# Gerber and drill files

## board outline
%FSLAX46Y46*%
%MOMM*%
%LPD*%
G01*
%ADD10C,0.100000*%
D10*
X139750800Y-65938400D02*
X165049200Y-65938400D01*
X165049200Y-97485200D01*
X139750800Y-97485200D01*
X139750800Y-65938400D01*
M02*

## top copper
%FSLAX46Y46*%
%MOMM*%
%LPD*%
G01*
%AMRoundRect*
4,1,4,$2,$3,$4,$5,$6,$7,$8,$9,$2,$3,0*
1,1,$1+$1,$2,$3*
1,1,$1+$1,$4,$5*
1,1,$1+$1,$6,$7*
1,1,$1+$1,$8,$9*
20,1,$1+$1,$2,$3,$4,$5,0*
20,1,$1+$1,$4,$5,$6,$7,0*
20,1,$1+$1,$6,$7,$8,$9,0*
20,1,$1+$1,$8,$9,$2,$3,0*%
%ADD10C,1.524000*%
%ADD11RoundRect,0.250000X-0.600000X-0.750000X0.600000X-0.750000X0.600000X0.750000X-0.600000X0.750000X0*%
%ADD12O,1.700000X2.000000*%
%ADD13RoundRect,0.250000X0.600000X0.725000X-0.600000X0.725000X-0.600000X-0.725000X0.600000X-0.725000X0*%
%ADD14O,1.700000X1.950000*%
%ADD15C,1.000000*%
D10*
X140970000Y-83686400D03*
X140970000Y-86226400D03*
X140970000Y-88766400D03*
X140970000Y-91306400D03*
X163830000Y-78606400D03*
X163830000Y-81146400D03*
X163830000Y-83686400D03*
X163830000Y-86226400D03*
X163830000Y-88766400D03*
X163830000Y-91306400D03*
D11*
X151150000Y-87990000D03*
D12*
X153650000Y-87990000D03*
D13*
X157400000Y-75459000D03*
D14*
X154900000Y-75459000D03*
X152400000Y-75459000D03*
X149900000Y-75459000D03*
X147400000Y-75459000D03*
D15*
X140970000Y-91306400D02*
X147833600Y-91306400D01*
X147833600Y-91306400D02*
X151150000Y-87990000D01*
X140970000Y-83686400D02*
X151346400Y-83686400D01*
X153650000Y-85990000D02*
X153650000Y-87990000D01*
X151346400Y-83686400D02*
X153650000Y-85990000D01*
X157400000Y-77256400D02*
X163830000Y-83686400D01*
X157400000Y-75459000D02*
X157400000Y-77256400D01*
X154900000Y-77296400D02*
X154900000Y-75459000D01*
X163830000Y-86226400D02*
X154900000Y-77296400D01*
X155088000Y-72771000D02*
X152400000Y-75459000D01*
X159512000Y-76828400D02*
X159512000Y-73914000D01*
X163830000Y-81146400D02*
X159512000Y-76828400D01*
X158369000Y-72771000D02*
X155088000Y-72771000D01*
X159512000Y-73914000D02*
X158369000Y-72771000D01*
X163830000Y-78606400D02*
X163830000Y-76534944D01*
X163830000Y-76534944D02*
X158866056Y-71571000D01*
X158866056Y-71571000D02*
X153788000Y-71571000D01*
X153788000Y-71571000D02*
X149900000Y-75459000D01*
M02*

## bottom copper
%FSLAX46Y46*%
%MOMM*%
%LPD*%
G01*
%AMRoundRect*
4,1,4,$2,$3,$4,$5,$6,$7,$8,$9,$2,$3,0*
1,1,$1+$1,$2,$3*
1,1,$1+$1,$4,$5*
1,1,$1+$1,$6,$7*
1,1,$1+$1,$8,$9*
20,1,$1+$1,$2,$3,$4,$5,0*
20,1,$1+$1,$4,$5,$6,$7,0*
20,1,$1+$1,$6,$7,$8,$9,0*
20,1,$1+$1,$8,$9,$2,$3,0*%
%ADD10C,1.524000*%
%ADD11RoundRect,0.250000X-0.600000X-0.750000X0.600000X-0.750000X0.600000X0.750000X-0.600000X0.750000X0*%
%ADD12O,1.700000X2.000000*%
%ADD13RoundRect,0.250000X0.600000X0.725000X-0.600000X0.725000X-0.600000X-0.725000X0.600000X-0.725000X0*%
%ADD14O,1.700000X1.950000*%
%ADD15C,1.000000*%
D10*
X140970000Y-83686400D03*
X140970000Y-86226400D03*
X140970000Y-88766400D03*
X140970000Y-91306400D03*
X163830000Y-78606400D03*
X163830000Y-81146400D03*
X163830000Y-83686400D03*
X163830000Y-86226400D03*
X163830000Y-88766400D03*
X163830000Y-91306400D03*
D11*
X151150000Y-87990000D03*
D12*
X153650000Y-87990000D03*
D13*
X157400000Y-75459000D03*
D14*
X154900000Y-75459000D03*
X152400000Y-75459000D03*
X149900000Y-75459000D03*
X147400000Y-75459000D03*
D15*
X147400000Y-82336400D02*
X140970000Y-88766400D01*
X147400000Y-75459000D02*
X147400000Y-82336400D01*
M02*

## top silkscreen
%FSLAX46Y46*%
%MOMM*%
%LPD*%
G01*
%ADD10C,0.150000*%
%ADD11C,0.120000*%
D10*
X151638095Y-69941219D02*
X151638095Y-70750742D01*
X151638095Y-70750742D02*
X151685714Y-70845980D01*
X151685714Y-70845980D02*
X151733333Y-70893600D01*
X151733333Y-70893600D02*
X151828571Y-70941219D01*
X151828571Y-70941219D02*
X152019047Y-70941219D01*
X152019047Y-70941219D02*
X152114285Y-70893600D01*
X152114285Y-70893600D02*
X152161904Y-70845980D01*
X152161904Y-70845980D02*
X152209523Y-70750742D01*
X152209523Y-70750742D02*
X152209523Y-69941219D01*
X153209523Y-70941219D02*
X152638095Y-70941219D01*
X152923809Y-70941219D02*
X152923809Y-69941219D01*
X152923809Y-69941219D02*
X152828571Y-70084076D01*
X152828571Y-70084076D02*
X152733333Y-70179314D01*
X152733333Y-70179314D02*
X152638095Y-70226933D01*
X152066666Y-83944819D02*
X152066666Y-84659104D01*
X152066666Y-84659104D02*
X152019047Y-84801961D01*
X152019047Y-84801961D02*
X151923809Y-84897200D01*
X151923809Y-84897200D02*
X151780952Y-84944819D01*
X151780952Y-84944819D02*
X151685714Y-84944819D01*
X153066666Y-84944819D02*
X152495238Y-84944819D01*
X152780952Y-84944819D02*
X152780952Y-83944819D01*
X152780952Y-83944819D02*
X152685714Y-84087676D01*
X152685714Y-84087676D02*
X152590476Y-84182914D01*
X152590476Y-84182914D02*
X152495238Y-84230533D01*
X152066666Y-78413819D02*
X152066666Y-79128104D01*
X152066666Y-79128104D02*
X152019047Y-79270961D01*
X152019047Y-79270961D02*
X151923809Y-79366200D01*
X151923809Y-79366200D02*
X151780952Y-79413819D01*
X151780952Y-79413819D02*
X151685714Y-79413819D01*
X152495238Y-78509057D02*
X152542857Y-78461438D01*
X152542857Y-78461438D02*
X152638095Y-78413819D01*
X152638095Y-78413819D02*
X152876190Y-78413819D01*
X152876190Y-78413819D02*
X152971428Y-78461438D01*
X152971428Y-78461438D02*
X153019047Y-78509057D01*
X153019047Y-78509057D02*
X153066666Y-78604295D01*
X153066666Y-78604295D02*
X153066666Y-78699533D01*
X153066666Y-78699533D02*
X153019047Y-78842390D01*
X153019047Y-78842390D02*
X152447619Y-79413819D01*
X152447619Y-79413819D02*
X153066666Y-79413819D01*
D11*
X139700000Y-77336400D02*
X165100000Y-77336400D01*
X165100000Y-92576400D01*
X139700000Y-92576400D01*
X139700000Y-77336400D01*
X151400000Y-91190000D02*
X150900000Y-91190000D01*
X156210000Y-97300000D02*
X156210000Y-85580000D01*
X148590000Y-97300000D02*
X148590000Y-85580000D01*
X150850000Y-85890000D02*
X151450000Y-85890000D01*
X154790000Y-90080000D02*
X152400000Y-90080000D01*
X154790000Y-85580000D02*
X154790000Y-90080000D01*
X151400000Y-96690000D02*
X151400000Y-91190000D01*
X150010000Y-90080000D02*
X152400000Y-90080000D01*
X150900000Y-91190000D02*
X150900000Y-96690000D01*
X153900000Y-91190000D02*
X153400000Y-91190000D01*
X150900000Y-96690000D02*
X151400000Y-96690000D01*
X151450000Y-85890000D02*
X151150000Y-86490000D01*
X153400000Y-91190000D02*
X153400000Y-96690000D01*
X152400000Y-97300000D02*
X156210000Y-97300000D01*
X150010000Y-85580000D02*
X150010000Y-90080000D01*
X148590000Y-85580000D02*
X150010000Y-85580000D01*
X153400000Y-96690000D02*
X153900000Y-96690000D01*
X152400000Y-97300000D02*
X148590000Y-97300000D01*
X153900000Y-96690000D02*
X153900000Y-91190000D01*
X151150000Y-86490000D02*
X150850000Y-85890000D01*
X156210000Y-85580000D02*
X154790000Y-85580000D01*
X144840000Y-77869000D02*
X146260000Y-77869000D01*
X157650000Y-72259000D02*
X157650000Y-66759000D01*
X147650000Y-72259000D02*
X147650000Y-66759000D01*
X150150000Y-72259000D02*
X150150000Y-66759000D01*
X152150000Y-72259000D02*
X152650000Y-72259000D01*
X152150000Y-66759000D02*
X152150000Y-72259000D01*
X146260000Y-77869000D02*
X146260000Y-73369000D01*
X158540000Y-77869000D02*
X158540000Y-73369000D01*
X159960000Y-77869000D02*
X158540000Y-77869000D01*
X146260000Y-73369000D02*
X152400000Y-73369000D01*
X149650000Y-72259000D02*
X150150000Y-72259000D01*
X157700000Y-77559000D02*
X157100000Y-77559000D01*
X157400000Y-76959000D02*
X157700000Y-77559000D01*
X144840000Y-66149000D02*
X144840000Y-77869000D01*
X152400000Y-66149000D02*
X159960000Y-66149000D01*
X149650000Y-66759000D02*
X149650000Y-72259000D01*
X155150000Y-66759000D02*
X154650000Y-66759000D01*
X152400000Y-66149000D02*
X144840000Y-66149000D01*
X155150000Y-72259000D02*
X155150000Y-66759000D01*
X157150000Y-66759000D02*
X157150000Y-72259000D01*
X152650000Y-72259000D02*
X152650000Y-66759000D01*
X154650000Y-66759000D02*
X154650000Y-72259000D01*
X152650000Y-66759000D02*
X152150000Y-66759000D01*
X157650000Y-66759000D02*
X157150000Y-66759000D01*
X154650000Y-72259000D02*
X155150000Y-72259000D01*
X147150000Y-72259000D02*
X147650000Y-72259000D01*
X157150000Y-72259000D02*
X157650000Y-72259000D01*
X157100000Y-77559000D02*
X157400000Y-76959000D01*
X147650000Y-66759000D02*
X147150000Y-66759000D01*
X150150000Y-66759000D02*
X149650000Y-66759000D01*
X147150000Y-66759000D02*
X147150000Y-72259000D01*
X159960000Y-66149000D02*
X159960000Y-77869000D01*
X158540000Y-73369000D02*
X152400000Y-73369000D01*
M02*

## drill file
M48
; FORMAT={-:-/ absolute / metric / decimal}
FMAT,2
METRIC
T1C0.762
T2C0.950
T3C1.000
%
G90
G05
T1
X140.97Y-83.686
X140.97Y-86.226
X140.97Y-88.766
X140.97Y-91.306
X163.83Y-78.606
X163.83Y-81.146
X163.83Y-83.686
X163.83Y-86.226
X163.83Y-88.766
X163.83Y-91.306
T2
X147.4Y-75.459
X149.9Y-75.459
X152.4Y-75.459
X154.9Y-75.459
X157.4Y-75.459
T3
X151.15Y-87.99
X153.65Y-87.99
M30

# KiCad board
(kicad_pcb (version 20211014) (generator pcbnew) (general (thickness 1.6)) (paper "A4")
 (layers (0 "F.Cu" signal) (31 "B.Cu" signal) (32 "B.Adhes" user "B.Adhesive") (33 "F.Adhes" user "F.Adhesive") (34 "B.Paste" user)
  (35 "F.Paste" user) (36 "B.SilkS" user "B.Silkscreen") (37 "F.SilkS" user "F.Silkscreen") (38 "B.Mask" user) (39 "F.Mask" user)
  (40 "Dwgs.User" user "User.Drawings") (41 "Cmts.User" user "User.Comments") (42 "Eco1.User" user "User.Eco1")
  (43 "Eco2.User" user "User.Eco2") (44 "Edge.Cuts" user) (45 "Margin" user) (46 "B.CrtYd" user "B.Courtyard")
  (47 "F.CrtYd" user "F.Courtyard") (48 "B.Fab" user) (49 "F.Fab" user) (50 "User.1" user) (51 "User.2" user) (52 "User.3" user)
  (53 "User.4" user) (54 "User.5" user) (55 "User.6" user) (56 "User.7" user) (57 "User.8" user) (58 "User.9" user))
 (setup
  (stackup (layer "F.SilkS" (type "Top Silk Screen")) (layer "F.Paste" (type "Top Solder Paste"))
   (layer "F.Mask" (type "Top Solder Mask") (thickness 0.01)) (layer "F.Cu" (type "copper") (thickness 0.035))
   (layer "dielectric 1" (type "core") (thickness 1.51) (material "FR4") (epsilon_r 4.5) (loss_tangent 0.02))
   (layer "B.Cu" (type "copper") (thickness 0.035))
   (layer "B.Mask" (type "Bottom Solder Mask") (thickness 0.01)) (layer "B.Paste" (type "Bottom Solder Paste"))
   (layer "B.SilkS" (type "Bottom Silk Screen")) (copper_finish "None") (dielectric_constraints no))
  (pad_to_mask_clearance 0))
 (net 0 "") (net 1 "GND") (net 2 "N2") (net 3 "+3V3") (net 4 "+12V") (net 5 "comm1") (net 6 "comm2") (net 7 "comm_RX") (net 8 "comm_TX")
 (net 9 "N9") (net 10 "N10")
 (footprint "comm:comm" (layer "F.Cu") (at 152.4 70.9864)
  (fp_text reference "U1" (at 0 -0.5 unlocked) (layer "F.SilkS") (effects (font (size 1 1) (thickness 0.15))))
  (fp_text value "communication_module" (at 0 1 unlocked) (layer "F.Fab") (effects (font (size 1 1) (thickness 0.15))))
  (fp_rect (start -12.7 21.59) (end 12.7 6.35) (layer "F.SilkS") (width 0.12) (fill none))
  (pad "1" thru_hole circle (at -11.43 12.7) (size 1.524 1.524) (drill 0.762) (layers *.Cu *.Mask) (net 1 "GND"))
  (pad "2" thru_hole circle (at -11.43 15.24) (size 1.524 1.524) (drill 0.762) (layers *.Cu *.Mask) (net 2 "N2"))
  (pad "3" thru_hole circle (at -11.43 17.78) (size 1.524 1.524) (drill 0.762) (layers *.Cu *.Mask) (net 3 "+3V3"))
  (pad "4" thru_hole circle (at -11.43 20.32) (size 1.524 1.524) (drill 0.762) (layers *.Cu *.Mask) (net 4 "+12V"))
  (pad "5" thru_hole circle (at 11.43 7.62) (size 1.524 1.524) (drill 0.762) (layers *.Cu *.Mask) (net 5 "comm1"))
  (pad "6" thru_hole circle (at 11.43 10.16) (size 1.524 1.524) (drill 0.762) (layers *.Cu *.Mask) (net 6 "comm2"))
  (pad "7" thru_hole circle (at 11.43 12.7) (size 1.524 1.524) (drill 0.762) (layers *.Cu *.Mask) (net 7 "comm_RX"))
  (pad "8" thru_hole circle (at 11.43 15.24) (size 1.524 1.524) (drill 0.762) (layers *.Cu *.Mask) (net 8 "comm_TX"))
  (pad "9" thru_hole circle (at 11.43 17.78) (size 1.524 1.524) (drill 0.762) (layers *.Cu *.Mask) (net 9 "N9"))
  (pad "10" thru_hole circle (at 11.43 20.32) (size 1.524 1.524) (drill 0.762) (layers *.Cu *.Mask) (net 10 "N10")))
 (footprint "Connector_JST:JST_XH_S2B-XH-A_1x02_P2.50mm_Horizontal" (layer "F.Cu") (at 151.15 87.99)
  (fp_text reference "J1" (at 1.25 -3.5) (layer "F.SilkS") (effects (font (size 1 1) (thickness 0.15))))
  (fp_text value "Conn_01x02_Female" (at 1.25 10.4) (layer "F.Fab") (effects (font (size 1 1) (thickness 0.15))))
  (fp_line (start 0.25 3.2) (end -0.25 3.2) (layer "F.SilkS") (width 0.12))
  (fp_line (start 5.06 9.31) (end 5.06 -2.41) (layer "F.SilkS") (width 0.12))
  (fp_line (start -2.56 9.31) (end -2.56 -2.41) (layer "F.SilkS") (width 0.12))
  (fp_line (start -0.3 -2.1) (end 0.3 -2.1) (layer "F.SilkS") (width 0.12))
  (fp_line (start 3.64 2.09) (end 1.25 2.09) (layer "F.SilkS") (width 0.12))
  (fp_line (start 3.64 -2.41) (end 3.64 2.09) (layer "F.SilkS") (width 0.12))
  (fp_line (start 0.25 8.7) (end 0.25 3.2) (layer "F.SilkS") (width 0.12))
  (fp_line (start -1.14 2.09) (end 1.25 2.09) (layer "F.SilkS") (width 0.12))
  (fp_line (start -0.25 3.2) (end -0.25 8.7) (layer "F.SilkS") (width 0.12))
  (fp_line (start 2.75 3.2) (end 2.25 3.2) (layer "F.SilkS") (width 0.12))
  (fp_line (start -0.25 8.7) (end 0.25 8.7) (layer "F.SilkS") (width 0.12))
  (fp_line (start 0.3 -2.1) (end 0 -1.5) (layer "F.SilkS") (width 0.12))
  (fp_line (start 2.25 3.2) (end 2.25 8.7) (layer "F.SilkS") (width 0.12))
  (fp_line (start 1.25 9.31) (end 5.06 9.31) (layer "F.SilkS") (width 0.12))
  (fp_line (start -1.14 -2.41) (end -1.14 2.09) (layer "F.SilkS") (width 0.12))
  (fp_line (start -2.56 -2.41) (end -1.14 -2.41) (layer "F.SilkS") (width 0.12))
  (fp_line (start 2.25 8.7) (end 2.75 8.7) (layer "F.SilkS") (width 0.12))
  (fp_line (start 1.25 9.31) (end -2.56 9.31) (layer "F.SilkS") (width 0.12))
  (fp_line (start 2.75 8.7) (end 2.75 3.2) (layer "F.SilkS") (width 0.12))
  (fp_line (start 0 -1.5) (end -0.3 -2.1) (layer "F.SilkS") (width 0.12))
  (fp_line (start 5.06 -2.41) (end 3.64 -2.41) (layer "F.SilkS") (width 0.12))
  (pad "1" thru_hole roundrect (at 0 0) (size 1.7 2) (drill 1) (layers *.Cu *.Mask) (roundrect_rratio 0.147059) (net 4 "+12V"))
  (pad "2" thru_hole oval (at 2.5 0) (size 1.7 2) (drill 1) (layers *.Cu *.Mask) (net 1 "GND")))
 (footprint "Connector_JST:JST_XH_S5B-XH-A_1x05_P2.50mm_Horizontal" (layer "F.Cu") (at 157.4 75.459 180)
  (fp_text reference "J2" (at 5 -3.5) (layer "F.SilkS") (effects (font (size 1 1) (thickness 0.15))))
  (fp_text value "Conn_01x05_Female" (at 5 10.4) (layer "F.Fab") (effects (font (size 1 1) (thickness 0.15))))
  (fp_line (start 12.56 -2.41) (end 11.14 -2.41) (layer "F.SilkS") (width 0.12))
  (fp_line (start -0.25 3.2) (end -0.25 8.7) (layer "F.SilkS") (width 0.12))
  (fp_line (start 9.75 3.2) (end 9.75 8.7) (layer "F.SilkS") (width 0.12))
  (fp_line (start 7.25 3.2) (end 7.25 8.7) (layer "F.SilkS") (width 0.12))
  (fp_line (start 5.25 3.2) (end 4.75 3.2) (layer "F.SilkS") (width 0.12))
  (fp_line (start 5.25 8.7) (end 5.25 3.2) (layer "F.SilkS") (width 0.12))
  (fp_line (start 11.14 -2.41) (end 11.14 2.09) (layer "F.SilkS") (width 0.12))
  (fp_line (start -1.14 -2.41) (end -1.14 2.09) (layer "F.SilkS") (width 0.12))
  (fp_line (start -2.56 -2.41) (end -1.14 -2.41) (layer "F.SilkS") (width 0.12))
  (fp_line (start 11.14 2.09) (end 5 2.09) (layer "F.SilkS") (width 0.12))
  (fp_line (start 7.75 3.2) (end 7.25 3.2) (layer "F.SilkS") (width 0.12))
  (fp_line (start -0.3 -2.1) (end 0.3 -2.1) (layer "F.SilkS") (width 0.12))
  (fp_line (start 0 -1.5) (end -0.3 -2.1) (layer "F.SilkS") (width 0.12))
  (fp_line (start 12.56 9.31) (end 12.56 -2.41) (layer "F.SilkS") (width 0.12))
  (fp_line (start 5 9.31) (end -2.56 9.31) (layer "F.SilkS") (width 0.12))
  (fp_line (start 7.75 8.7) (end 7.75 3.2) (layer "F.SilkS") (width 0.12))
  (fp_line (start 2.25 8.7) (end 2.75 8.7) (layer "F.SilkS") (width 0.12))
  (fp_line (start 5 9.31) (end 12.56 9.31) (layer "F.SilkS") (width 0.12))
  (fp_line (start 2.25 3.2) (end 2.25 8.7) (layer "F.SilkS") (width 0.12))
  (fp_line (start 0.25 8.7) (end 0.25 3.2) (layer "F.SilkS") (width 0.12))
  (fp_line (start 4.75 3.2) (end 4.75 8.7) (layer "F.SilkS") (width 0.12))
  (fp_line (start 2.75 8.7) (end 2.75 3.2) (layer "F.SilkS") (width 0.12))
  (fp_line (start 4.75 8.7) (end 5.25 8.7) (layer "F.SilkS") (width 0.12))
  (fp_line (start -0.25 8.7) (end 0.25 8.7) (layer "F.SilkS") (width 0.12))
  (fp_line (start 2.75 3.2) (end 2.25 3.2) (layer "F.SilkS") (width 0.12))
  (fp_line (start 10.25 3.2) (end 9.75 3.2) (layer "F.SilkS") (width 0.12))
  (fp_line (start 0.25 3.2) (end -0.25 3.2) (layer "F.SilkS") (width 0.12))
  (fp_line (start 0.3 -2.1) (end 0 -1.5) (layer "F.SilkS") (width 0.12))
  (fp_line (start 9.75 8.7) (end 10.25 8.7) (layer "F.SilkS") (width 0.12))
  (fp_line (start 7.25 8.7) (end 7.75 8.7) (layer "F.SilkS") (width 0.12))
  (fp_line (start 10.25 8.7) (end 10.25 3.2) (layer "F.SilkS") (width 0.12))
  (fp_line (start -2.56 9.31) (end -2.56 -2.41) (layer "F.SilkS") (width 0.12))
  (fp_line (start -1.14 2.09) (end 5 2.09) (layer "F.SilkS") (width 0.12))
  (pad "1" thru_hole roundrect (at 0 0 180) (size 1.7 1.95) (drill 0.95) (layers *.Cu *.Mask) (roundrect_rratio 0.147059) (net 7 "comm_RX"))
  (pad "2" thru_hole oval (at 2.5 0 180) (size 1.7 1.95) (drill 0.95) (layers *.Cu *.Mask) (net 8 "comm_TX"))
  (pad "3" thru_hole oval (at 5 0 180) (size 1.7 1.95) (drill 0.95) (layers *.Cu *.Mask) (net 6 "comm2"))
  (pad "4" thru_hole oval (at 7.5 0 180) (size 1.7 1.95) (drill 0.95) (layers *.Cu *.Mask) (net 5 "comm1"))
  (pad "5" thru_hole oval (at 10 0 180) (size 1.7 1.95) (drill 0.95) (layers *.Cu *.Mask) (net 3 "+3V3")))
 (gr_rect (start 139.7508 97.4852) (end 165.0492 65.9384) (layer "Edge.Cuts") (width 0.1) (fill none))
 (segment (start 140.97 91.3064) (end 147.8336 91.3064) (width 1) (layer "F.Cu") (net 4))
 (segment (start 147.8336 91.3064) (end 151.15 87.99) (width 1) (layer "F.Cu") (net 4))
 (segment (start 140.97 83.6864) (end 151.3464 83.6864) (width 1) (layer "F.Cu") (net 1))
 (segment (start 153.65 85.99) (end 153.65 87.99) (width 1) (layer "F.Cu") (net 1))
 (segment (start 151.3464 83.6864) (end 153.65 85.99) (width 1) (layer "F.Cu") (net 1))
 (segment (start 157.4 77.2564) (end 163.83 83.6864) (width 1) (layer "F.Cu") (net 7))
 (segment (start 157.4 75.459) (end 157.4 77.2564) (width 1) (layer "F.Cu") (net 7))
 (segment (start 154.9 77.2964) (end 154.9 75.459) (width 1) (layer "F.Cu") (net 8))
 (segment (start 163.83 86.2264) (end 154.9 77.2964) (width 1) (layer "F.Cu") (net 8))
 (segment (start 155.088 72.771) (end 152.4 75.459) (width 1) (layer "F.Cu") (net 6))
 (segment (start 159.512 76.8284) (end 159.512 73.914) (width 1) (layer "F.Cu") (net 6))
 (segment (start 163.83 81.1464) (end 159.512 76.8284) (width 1) (layer "F.Cu") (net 6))
 (segment (start 158.369 72.771) (end 155.088 72.771) (width 1) (layer "F.Cu") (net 6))
 (segment (start 159.512 73.914) (end 158.369 72.771) (width 1) (layer "F.Cu") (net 6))
 (segment (start 163.83 78.6064) (end 163.83 76.534944) (width 1) (layer "F.Cu") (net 5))
 (segment (start 163.83 76.534944) (end 158.866056 71.571) (width 1) (layer "F.Cu") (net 5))
 (segment (start 158.866056 71.571) (end 153.788 71.571) (width 1) (layer "F.Cu") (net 5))
 (segment (start 153.788 71.571) (end 149.9 75.459) (width 1) (layer "F.Cu") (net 5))
 (segment (start 147.4 82.3364) (end 140.97 88.7664) (width 1) (layer "B.Cu") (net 3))
 (segment (start 147.4 75.459) (end 147.4 82.3364) (width 1) (layer "B.Cu") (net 3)))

